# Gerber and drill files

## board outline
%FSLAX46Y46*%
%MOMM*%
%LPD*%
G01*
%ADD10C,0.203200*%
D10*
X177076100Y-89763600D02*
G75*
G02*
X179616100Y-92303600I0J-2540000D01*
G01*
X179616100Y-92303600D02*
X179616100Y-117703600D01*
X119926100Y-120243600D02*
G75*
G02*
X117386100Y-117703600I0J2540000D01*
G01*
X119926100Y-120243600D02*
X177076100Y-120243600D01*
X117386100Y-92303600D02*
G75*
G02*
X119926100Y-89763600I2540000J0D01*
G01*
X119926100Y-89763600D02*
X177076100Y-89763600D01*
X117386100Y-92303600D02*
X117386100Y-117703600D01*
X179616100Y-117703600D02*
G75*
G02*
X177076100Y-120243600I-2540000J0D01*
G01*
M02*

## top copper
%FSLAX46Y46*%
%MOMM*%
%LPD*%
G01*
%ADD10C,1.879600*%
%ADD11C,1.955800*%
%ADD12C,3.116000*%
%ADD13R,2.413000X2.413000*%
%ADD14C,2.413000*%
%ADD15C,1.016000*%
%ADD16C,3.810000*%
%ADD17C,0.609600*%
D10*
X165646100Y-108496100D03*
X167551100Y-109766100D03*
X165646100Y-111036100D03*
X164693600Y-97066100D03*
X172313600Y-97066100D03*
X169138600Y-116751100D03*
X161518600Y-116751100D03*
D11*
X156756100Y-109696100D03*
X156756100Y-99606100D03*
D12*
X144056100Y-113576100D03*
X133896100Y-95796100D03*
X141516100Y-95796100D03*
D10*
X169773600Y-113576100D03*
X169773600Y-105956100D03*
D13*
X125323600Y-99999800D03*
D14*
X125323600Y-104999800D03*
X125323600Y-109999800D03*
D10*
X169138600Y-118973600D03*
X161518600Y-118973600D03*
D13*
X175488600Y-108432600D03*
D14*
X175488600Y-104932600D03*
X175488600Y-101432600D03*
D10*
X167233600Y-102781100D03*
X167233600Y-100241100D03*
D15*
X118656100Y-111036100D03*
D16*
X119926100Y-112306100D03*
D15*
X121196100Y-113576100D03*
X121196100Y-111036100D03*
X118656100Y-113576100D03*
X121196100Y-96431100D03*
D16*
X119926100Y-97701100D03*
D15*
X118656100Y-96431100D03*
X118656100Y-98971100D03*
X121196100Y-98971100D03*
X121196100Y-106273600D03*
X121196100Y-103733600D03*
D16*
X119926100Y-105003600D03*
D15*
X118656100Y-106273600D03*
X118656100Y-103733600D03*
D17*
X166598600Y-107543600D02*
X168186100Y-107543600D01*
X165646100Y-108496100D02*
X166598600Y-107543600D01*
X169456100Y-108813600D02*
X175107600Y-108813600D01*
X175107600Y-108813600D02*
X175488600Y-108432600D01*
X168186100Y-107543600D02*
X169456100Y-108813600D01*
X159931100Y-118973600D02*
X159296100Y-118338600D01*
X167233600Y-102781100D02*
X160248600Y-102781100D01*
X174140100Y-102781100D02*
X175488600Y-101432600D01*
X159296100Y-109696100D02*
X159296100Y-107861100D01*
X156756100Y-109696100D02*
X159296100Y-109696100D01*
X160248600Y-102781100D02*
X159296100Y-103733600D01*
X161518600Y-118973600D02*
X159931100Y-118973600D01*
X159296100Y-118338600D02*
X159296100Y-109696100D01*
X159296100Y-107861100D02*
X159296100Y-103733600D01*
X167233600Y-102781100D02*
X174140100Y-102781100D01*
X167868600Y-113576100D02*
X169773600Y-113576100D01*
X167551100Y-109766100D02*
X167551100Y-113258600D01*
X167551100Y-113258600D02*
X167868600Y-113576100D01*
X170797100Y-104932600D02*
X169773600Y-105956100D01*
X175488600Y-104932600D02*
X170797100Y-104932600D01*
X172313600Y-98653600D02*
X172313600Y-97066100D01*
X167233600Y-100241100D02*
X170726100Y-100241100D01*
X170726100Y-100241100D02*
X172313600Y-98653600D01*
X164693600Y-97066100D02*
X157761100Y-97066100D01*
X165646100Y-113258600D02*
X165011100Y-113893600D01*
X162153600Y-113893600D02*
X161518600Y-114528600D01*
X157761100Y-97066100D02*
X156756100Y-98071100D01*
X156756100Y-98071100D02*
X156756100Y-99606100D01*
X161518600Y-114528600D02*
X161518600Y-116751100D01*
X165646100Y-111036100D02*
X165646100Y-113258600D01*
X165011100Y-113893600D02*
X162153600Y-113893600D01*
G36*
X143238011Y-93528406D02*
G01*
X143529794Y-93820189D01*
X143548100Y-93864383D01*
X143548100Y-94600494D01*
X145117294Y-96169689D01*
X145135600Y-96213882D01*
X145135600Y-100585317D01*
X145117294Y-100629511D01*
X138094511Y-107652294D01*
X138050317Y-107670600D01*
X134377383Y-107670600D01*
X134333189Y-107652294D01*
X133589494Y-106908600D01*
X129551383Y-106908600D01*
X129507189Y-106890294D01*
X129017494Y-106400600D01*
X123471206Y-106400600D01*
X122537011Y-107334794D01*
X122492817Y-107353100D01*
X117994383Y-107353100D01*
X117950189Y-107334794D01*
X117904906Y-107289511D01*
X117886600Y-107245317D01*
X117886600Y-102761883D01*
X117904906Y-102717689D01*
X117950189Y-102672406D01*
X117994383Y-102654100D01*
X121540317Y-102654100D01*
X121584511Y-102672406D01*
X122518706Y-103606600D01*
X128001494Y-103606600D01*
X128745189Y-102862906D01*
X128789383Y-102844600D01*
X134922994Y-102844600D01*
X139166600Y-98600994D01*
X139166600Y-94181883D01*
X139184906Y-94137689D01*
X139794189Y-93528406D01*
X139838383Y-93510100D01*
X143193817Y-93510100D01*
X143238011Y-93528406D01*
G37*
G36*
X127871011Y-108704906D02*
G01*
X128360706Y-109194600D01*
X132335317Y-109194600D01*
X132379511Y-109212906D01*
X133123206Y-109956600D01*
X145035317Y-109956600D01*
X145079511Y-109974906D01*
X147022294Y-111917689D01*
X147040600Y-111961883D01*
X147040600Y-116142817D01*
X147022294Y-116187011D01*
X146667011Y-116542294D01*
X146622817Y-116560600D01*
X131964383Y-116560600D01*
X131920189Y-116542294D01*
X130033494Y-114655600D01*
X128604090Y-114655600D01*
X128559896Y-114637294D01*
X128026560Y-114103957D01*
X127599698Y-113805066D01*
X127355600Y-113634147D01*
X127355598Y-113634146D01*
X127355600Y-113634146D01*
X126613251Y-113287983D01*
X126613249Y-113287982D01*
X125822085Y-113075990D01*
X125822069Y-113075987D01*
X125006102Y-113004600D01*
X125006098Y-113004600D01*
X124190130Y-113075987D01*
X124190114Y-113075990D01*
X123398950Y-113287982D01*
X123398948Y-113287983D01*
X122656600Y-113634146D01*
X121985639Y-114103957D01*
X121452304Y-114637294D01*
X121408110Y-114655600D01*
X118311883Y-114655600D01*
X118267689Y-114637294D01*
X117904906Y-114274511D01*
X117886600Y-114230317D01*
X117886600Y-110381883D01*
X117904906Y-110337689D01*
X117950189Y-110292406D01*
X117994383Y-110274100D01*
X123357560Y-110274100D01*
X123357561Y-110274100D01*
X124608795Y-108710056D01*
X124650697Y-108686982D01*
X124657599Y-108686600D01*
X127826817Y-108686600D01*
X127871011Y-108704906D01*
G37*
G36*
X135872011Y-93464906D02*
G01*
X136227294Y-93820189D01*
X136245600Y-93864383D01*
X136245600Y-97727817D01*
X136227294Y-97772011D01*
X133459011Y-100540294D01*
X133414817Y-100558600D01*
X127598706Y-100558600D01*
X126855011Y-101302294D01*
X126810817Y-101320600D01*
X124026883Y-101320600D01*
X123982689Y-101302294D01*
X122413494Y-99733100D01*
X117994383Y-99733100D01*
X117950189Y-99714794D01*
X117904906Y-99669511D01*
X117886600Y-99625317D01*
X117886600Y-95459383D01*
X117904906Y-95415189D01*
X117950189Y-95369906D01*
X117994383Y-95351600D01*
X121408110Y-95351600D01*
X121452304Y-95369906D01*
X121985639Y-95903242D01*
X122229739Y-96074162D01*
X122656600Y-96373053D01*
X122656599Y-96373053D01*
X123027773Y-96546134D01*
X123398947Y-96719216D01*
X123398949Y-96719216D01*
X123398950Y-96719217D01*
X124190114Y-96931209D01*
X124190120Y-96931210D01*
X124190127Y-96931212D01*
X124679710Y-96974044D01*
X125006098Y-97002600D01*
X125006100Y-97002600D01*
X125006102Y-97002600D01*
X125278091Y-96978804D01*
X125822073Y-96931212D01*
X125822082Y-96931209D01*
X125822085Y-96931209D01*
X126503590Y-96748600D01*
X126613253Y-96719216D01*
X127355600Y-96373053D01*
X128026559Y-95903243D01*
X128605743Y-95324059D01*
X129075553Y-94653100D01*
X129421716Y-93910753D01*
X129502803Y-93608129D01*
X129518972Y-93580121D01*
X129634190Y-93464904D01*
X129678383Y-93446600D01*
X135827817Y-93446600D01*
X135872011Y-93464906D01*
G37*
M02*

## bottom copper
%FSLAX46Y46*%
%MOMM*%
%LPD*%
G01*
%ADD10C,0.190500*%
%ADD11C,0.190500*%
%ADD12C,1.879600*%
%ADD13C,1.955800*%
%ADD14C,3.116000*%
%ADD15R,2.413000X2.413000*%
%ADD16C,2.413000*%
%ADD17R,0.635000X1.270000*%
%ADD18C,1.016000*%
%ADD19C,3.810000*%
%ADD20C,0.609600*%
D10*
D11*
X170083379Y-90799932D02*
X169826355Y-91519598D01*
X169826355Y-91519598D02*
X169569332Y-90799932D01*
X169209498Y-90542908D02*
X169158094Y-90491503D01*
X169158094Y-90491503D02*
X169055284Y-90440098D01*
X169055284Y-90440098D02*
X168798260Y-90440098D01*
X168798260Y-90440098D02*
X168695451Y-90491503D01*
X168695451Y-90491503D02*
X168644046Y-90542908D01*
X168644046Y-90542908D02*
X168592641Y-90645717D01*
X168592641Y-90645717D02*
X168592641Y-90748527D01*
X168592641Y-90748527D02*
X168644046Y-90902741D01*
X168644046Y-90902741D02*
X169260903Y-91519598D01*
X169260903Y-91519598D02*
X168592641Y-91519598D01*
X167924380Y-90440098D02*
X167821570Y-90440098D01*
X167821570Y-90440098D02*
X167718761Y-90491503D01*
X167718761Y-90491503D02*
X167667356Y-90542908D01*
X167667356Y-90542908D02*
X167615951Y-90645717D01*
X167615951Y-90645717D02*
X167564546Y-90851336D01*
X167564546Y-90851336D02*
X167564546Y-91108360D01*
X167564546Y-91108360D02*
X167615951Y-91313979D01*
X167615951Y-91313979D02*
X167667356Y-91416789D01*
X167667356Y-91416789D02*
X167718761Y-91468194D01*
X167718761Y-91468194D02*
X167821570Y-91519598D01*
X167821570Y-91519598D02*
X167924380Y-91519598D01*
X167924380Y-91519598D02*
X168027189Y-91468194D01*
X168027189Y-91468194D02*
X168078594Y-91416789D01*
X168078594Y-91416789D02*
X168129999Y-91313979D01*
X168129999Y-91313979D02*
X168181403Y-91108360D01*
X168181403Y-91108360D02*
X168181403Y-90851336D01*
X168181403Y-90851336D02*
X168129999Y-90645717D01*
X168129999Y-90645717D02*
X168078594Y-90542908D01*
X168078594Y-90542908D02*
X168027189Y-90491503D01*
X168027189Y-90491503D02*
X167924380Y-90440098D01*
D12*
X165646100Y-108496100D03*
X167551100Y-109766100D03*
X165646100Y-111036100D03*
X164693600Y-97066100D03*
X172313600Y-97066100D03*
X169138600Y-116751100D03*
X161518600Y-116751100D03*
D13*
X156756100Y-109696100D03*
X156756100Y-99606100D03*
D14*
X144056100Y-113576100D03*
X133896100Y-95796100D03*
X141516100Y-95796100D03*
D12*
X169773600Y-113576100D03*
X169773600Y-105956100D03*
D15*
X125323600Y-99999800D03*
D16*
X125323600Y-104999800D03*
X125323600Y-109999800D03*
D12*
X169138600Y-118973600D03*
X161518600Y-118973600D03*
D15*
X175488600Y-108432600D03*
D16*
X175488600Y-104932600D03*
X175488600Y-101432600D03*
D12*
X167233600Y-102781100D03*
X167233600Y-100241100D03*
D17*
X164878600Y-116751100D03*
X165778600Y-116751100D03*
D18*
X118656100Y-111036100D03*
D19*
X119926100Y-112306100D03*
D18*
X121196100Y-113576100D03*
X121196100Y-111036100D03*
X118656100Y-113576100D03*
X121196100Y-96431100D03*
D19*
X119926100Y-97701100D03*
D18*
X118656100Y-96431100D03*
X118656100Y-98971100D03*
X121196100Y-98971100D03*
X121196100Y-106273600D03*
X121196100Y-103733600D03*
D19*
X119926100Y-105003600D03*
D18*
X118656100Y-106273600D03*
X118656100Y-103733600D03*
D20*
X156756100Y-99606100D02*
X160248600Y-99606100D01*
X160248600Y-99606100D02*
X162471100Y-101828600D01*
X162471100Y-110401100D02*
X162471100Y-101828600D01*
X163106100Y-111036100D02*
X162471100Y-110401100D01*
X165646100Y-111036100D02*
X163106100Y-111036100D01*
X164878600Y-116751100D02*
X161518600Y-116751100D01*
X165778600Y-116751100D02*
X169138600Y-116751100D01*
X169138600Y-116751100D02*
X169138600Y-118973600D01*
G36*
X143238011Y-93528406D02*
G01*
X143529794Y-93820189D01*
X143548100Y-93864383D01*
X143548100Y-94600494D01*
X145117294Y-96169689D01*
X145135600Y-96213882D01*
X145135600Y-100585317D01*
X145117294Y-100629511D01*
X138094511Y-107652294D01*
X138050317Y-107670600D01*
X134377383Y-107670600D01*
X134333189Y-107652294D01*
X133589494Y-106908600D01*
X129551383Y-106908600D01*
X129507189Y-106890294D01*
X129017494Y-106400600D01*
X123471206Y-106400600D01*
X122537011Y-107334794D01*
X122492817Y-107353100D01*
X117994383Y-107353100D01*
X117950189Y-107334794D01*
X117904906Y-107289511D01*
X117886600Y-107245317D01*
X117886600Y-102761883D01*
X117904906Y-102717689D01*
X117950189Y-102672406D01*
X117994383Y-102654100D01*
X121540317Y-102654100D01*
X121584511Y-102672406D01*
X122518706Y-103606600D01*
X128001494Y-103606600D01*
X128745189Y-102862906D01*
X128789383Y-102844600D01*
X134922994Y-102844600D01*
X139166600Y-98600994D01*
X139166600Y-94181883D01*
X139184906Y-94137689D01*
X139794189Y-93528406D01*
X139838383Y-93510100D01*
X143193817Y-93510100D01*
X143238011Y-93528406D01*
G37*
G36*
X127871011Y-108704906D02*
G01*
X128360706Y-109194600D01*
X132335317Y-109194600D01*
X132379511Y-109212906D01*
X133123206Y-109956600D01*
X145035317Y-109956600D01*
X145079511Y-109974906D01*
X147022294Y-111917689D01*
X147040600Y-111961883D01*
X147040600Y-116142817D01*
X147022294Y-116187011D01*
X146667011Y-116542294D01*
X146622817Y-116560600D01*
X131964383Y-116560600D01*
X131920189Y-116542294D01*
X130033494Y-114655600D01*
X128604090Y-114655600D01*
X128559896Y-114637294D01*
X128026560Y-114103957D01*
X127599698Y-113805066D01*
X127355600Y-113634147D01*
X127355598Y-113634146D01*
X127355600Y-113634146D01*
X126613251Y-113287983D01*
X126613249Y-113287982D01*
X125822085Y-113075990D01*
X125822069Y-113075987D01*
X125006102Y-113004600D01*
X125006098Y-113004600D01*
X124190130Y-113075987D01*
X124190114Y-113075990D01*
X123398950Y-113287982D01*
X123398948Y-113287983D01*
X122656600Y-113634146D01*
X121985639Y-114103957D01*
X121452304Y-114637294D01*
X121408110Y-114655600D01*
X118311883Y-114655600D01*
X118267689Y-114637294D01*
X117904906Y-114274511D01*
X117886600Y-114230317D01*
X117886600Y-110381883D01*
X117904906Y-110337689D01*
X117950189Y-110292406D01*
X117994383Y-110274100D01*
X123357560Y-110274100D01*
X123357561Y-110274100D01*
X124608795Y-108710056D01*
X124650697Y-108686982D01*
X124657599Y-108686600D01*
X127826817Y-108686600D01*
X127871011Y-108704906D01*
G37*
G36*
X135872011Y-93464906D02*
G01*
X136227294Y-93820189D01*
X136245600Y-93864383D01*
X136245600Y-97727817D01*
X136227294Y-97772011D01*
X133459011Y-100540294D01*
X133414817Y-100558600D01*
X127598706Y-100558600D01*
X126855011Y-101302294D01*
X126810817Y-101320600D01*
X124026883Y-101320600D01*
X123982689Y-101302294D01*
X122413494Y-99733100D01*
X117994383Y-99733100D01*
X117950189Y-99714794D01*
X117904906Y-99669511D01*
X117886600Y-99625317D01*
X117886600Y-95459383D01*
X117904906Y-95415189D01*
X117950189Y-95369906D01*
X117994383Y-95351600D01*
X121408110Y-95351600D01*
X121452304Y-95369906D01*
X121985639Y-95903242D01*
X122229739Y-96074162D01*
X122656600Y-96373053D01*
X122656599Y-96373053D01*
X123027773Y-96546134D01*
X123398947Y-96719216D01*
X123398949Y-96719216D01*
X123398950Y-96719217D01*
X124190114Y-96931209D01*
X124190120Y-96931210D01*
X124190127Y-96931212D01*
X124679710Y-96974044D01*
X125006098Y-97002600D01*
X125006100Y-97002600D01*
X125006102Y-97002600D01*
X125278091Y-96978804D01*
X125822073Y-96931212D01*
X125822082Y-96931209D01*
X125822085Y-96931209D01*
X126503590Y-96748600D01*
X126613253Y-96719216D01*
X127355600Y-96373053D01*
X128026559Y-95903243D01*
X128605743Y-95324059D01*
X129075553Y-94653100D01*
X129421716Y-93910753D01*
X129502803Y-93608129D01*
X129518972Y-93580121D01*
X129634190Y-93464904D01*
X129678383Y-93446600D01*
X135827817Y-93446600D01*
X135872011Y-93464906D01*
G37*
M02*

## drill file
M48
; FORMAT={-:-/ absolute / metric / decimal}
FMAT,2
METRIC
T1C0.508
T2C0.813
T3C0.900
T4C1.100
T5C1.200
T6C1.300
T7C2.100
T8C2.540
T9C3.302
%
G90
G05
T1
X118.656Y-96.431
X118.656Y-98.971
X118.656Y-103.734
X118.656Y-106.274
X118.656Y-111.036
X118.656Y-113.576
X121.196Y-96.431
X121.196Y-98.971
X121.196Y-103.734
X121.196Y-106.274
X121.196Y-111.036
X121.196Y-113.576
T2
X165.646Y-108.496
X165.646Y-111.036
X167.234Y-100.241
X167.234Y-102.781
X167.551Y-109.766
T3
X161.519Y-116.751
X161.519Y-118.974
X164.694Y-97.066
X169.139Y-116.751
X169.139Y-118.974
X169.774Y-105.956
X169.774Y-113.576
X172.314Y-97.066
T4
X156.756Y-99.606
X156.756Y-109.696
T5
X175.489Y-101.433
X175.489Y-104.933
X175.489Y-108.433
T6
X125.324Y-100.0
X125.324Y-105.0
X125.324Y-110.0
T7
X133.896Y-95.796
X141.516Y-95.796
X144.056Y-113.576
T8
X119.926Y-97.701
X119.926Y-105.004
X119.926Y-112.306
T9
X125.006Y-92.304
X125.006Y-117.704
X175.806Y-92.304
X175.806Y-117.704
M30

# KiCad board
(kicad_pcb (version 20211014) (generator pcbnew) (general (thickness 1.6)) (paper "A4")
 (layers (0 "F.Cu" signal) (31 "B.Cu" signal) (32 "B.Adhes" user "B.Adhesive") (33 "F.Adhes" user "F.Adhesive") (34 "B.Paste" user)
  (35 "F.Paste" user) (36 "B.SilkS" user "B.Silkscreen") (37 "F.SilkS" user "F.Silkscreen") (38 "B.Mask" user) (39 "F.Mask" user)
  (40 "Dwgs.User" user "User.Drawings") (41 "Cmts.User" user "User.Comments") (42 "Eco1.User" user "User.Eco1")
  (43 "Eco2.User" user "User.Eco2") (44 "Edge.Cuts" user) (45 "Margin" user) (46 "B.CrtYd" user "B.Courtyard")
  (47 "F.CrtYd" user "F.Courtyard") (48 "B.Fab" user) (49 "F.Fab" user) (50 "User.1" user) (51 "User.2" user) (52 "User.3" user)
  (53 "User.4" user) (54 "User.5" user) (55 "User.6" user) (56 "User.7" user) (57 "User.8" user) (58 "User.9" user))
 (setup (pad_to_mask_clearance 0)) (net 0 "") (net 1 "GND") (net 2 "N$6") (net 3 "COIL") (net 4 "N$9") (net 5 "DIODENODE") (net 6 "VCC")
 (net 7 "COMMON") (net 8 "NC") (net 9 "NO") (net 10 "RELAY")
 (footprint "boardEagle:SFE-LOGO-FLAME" (layer "F.Cu") (at 167.8686 94.2086)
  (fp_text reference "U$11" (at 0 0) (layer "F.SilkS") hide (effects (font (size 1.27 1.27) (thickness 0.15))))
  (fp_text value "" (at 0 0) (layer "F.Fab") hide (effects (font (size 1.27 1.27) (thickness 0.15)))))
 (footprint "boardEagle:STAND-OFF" (layer "F.Cu") (at 125.0061 117.7036)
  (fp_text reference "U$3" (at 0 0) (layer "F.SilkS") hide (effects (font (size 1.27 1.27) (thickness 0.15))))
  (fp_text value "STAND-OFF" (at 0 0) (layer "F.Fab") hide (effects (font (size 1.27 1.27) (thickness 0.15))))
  (pad "" np_thru_hole circle (at 0 0) (size 3.302 3.302) (drill 3.302) (layers *.Cu *.Mask)))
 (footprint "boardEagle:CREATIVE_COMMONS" (layer "F.Cu") (at 116.2431 133.3246)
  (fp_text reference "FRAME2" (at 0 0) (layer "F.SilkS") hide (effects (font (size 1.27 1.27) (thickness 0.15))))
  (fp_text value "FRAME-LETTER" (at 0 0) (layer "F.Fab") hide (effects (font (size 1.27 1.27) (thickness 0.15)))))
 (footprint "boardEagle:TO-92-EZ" (layer "F.Cu") (at 165.6461 109.7661 -90)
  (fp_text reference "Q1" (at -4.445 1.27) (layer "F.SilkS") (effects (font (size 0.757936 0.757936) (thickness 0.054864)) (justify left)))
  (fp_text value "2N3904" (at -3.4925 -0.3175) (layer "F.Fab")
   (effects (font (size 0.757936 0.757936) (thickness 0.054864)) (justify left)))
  (pad "1" thru_hole circle (at -1.27 0 270) (size 1.8796 1.8796) (drill 0.8128) (layers *.Cu) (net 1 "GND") (solder_mask_margin 0.1016))
  (pad "2" thru_hole circle (at 0 -1.905 270) (size 1.8796 1.8796) (drill 0.8128) (layers *.Cu) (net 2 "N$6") (solder_mask_margin 0.1016))
  (pad "3" thru_hole circle (at 1.27 0 270) (size 1.8796 1.8796) (drill 0.8128) (layers *.Cu) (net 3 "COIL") (solder_mask_margin 0.1016)))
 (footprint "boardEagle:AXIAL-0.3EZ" (layer "F.Cu") (at 168.5036 97.0661)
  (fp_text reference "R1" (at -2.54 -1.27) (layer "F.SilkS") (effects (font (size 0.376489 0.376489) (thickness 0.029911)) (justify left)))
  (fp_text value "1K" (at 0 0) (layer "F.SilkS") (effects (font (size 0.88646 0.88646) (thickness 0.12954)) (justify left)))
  (pad "P$1" thru_hole circle (at -3.81 0) (size 1.8796 1.8796) (drill 0.9) (layers *.Cu) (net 3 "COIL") (solder_mask_margin 0.1016))
  (pad "P$2" thru_hole circle (at 3.81 0) (size 1.8796 1.8796) (drill 0.9) (layers *.Cu) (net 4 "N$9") (solder_mask_margin 0.1016)))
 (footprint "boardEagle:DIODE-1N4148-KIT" (layer "F.Cu") (at 165.3286 116.7511 180)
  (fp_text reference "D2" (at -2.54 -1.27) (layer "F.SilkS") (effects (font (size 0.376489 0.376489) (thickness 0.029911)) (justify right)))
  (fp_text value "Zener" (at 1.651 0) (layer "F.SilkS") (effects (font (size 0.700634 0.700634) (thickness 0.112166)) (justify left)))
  (pad "A" thru_hole circle (at -3.81 0 180) (size 1.8796 1.8796) (drill 0.9) (layers *.Cu) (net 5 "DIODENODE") (solder_mask_margin 0.1016))
  (pad "C" thru_hole circle (at 3.81 0 180) (size 1.8796 1.8796) (drill 0.9) (layers *.Cu) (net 3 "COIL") (solder_mask_margin 0.1016)))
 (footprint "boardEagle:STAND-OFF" (layer "F.Cu") (at 175.8061 117.7036)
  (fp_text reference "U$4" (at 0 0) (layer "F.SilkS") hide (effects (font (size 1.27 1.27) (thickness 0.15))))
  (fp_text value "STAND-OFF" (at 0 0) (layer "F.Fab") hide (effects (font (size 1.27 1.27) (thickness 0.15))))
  (pad "" np_thru_hole circle (at 0 0) (size 3.302 3.302) (drill 3.302) (layers *.Cu *.Mask)))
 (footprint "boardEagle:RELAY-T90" (layer "F.Cu") (at 156.7561 95.7961)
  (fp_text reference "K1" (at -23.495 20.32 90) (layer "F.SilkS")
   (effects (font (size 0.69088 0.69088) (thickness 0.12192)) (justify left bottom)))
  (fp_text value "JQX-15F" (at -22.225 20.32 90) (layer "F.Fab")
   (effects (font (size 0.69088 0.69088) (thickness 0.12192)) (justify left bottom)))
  (pad "COIL1" thru_hole circle (at 0 13.9 90) (size 1.9558 1.9558) (drill 1.1) (layers *.Cu *.Mask) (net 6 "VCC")
   (solder_mask_margin 0.1016))
  (pad "COIL2" thru_hole circle (at 0 3.81 90) (size 1.9558 1.9558) (drill 1.1) (layers *.Cu *.Mask) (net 3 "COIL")
   (solder_mask_margin 0.1016))
  (pad "MAIN" thru_hole circle (at -12.7 17.78 90) (size 3.116 3.116) (drill 2.1) (layers *.Cu *.Mask) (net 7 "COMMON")
   (solder_mask_margin 0.1016))
  (pad "NC" thru_hole circle (at -22.86 0 90) (size 3.116 3.116) (drill 2.1) (layers *.Cu *.Mask) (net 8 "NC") (solder_mask_margin 0.1016))
  (pad "NO" thru_hole circle (at -15.24 0 90) (size 3.116 3.116) (drill 2.1) (layers *.Cu *.Mask) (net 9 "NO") (solder_mask_margin 0.1016)))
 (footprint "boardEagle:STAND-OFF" (layer "F.Cu") (at 175.8061 92.3036)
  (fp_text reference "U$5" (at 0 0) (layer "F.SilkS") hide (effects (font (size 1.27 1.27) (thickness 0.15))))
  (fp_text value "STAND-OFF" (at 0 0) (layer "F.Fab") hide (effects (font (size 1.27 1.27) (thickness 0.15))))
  (pad "" np_thru_hole circle (at 0 0) (size 3.302 3.302) (drill 3.302) (layers *.Cu *.Mask)))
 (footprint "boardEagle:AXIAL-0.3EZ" (layer "F.Cu") (at 169.7736 109.7661 90)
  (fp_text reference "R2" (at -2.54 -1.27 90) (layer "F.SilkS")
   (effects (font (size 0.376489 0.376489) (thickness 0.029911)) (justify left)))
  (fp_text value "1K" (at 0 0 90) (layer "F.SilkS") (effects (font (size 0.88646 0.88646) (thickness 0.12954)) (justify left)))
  (pad "P$1" thru_hole circle (at -3.81 0 90) (size 1.8796 1.8796) (drill 0.9) (layers *.Cu) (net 2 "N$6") (solder_mask_margin 0.1016))
  (pad "P$2" thru_hole circle (at 3.81 0 90) (size 1.8796 1.8796) (drill 0.9) (layers *.Cu) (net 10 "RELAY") (solder_mask_margin 0.1016)))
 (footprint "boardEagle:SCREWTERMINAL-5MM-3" (layer "F.Cu") (at 125.3236 99.9998 -90)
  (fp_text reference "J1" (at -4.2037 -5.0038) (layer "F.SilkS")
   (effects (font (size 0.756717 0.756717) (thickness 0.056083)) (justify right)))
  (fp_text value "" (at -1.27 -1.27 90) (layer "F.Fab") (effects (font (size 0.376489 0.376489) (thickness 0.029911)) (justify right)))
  (pad "1" thru_hole rect (at 0 0 270) (size 2.413 2.413) (drill 1.3) (layers *.Cu *.Mask) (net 8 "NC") (solder_mask_margin 0.1016))
  (pad "2" thru_hole circle (at 5 0 270) (size 2.413 2.413) (drill 1.3) (layers *.Cu *.Mask) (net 9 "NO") (solder_mask_margin 0.1016))
  (pad "3" thru_hole circle (at 10 0 270) (size 2.413 2.413) (drill 1.3) (layers *.Cu *.Mask) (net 7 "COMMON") (solder_mask_margin 0.1016)))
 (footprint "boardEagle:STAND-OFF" (layer "F.Cu") (at 125.0061 92.3036)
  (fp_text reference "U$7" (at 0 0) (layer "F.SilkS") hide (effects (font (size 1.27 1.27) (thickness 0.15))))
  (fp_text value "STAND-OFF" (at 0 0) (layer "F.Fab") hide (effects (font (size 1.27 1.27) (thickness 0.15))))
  (pad "" np_thru_hole circle (at 0 0) (size 3.302 3.302) (drill 3.302) (layers *.Cu *.Mask)))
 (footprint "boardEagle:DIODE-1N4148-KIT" (layer "F.Cu") (at 165.3286 118.9736 180)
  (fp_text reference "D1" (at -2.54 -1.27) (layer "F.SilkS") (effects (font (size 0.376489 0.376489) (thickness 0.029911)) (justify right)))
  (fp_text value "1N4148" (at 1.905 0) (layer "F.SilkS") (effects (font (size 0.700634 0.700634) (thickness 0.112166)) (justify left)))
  (pad "A" thru_hole circle (at -3.81 0 180) (size 1.8796 1.8796) (drill 0.9) (layers *.Cu) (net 5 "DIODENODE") (solder_mask_margin 0.1016))
  (pad "C" thru_hole circle (at 3.81 0 180) (size 1.8796 1.8796) (drill 0.9) (layers *.Cu) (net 6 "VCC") (solder_mask_margin 0.1016)))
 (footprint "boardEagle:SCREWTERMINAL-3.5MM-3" (layer "F.Cu") (at 175.4886 108.4326 90)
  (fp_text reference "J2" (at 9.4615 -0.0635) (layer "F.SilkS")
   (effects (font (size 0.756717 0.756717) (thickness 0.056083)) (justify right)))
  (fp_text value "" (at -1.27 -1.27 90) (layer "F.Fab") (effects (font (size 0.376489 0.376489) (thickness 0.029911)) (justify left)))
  (pad "1" thru_hole rect (at 0 0 90) (size 2.413 2.413) (drill 1.2) (layers *.Cu *.Mask) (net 1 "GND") (solder_mask_margin 0.1016))
  (pad "2" thru_hole circle (at 3.5 0 90) (size 2.413 2.413) (drill 1.2) (layers *.Cu *.Mask) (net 10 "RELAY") (solder_mask_margin 0.1016))
  (pad "3" thru_hole circle (at 7 0 90) (size 2.413 2.413) (drill 1.2) (layers *.Cu *.Mask) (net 6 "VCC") (solder_mask_margin 0.1016)))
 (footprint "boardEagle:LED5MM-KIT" (layer "F.Cu") (at 167.2336 101.5111 90)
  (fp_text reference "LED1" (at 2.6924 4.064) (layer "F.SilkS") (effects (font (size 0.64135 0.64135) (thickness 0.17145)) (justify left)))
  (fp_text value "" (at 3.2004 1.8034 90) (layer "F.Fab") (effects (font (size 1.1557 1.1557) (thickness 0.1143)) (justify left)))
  (pad "A" thru_hole circle (at -1.27 0 90) (size 1.8796 1.8796) (drill 0.8128) (layers *.Cu) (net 6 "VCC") (solder_mask_margin 0.1016))
  (pad "K" thru_hole circle (at 1.27 0 90) (size 1.8796 1.8796) (drill 0.8128) (layers *.Cu) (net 4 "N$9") (solder_mask_margin 0.1016)))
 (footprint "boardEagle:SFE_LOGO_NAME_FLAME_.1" (layer "B.Cu") (at 142.3416 117.3861 180)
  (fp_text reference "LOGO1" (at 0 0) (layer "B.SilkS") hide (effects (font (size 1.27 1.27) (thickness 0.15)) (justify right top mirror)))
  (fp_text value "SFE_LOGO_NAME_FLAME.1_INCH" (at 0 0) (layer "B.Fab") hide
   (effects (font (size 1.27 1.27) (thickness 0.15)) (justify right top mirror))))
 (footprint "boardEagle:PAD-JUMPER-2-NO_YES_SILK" (layer "B.Cu") (at 165.3286 116.7511)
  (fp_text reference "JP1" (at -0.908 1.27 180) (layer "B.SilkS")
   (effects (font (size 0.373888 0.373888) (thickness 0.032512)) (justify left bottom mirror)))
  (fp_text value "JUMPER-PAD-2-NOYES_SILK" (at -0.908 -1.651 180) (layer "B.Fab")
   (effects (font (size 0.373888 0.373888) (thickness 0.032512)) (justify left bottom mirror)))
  (pad "1" smd rect (at -0.45 0) (size 0.635 1.27) (layers "B.Cu" "B.Mask") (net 3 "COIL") (solder_mask_margin 0.1016))
  (pad "2" smd rect (at 0.45 0) (size 0.635 1.27) (layers "B.Cu" "B.Mask") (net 5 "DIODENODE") (solder_mask_margin 0.1016)))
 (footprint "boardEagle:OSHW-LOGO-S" (layer "B.Cu") (at 169.1386 93.5736 180)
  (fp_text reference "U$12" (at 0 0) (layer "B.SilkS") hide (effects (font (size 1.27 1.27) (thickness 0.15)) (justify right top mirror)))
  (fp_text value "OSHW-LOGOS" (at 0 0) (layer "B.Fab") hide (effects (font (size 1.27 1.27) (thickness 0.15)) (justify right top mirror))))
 (gr_arc (start 177.0761 89.7636) (mid 178.872151 90.507549) (end 179.6161 92.3036) (layer "Edge.Cuts") (width 0.2032))
 (gr_line (start 179.6161 92.3036) (end 179.6161 117.7036) (layer "Edge.Cuts") (width 0.2032))
 (gr_arc (start 119.9261 120.2436) (mid 118.130049 119.499651) (end 117.3861 117.7036) (layer "Edge.Cuts") (width 0.2032))
 (gr_line (start 119.9261 120.2436) (end 177.0761 120.2436) (layer "Edge.Cuts") (width 0.2032))
 (gr_arc (start 117.3861 92.3036) (mid 118.130049 90.507549) (end 119.9261 89.7636) (layer "Edge.Cuts") (width 0.2032))
 (gr_line (start 119.9261 89.7636) (end 177.0761 89.7636) (layer "Edge.Cuts") (width 0.2032))
 (gr_line (start 117.3861 92.3036) (end 117.3861 117.7036) (layer "Edge.Cuts") (width 0.2032))
 (gr_arc (start 179.6161 117.7036) (mid 178.872151 119.499651) (end 177.0761 120.2436) (layer "Edge.Cuts") (width 0.2032))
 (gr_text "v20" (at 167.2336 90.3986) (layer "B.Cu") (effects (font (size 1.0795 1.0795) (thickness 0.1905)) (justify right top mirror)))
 (segment (start 166.5986 107.5436) (end 168.1861 107.5436) (width 0.6096) (layer "F.Cu") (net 1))
 (segment (start 165.6461 108.4961) (end 166.5986 107.5436) (width 0.6096) (layer "F.Cu") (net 1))
 (segment (start 169.4561 108.8136) (end 175.1076 108.8136) (width 0.6096) (layer "F.Cu") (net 1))
 (segment (start 175.1076 108.8136) (end 175.4886 108.4326) (width 0.6096) (layer "F.Cu") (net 1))
 (segment (start 168.1861 107.5436) (end 169.4561 108.8136) (width 0.6096) (layer "F.Cu") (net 1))
 (segment (start 159.9311 118.9736) (end 159.2961 118.3386) (width 0.6096) (layer "F.Cu") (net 6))
 (segment (start 167.2336 102.7811) (end 160.2486 102.7811) (width 0.6096) (layer "F.Cu") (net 6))
 (segment (start 174.1401 102.7811) (end 175.4886 101.4326) (width 0.6096) (layer "F.Cu") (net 6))
 (segment (start 159.2961 109.6961) (end 159.2961 107.8611) (width 0.6096) (layer "F.Cu") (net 6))
 (segment (start 156.7561 109.6961) (end 159.2961 109.6961) (width 0.6096) (layer "F.Cu") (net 6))
 (segment (start 160.2486 102.7811) (end 159.2961 103.7336) (width 0.6096) (layer "F.Cu") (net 6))
 (segment (start 161.5186 118.9736) (end 159.9311 118.9736) (width 0.6096) (layer "F.Cu") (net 6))
 (segment (start 159.2961 118.3386) (end 159.2961 109.6961) (width 0.6096) (layer "F.Cu") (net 6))
 (segment (start 159.2961 107.8611) (end 159.2961 103.7336) (width 0.6096) (layer "F.Cu") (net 6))
 (segment (start 167.2336 102.7811) (end 174.1401 102.7811) (width 0.6096) (layer "F.Cu") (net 6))
 (segment (start 167.8686 113.5761) (end 169.7736 113.5761) (width 0.6096) (layer "F.Cu") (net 2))
 (segment (start 167.5511 109.7661) (end 167.5511 113.2586) (width 0.6096) (layer "F.Cu") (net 2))
 (segment (start 167.5511 113.2586) (end 167.8686 113.5761) (width 0.6096) (layer "F.Cu") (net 2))
 (segment (start 170.7971 104.9326) (end 169.7736 105.9561) (width 0.6096) (layer "F.Cu") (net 10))
 (segment (start 175.4886 104.9326) (end 170.7971 104.9326) (width 0.6096) (layer "F.Cu") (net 10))
 (segment (start 172.3136 98.6536) (end 172.3136 97.0661) (width 0.6096) (layer "F.Cu") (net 4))
 (segment (start 167.2336 100.2411) (end 170.7261 100.2411) (width 0.6096) (layer "F.Cu") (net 4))
 (segment (start 170.7261 100.2411) (end 172.3136 98.6536) (width 0.6096) (layer "F.Cu") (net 4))
 (segment (start 164.6936 97.0661) (end 157.7611 97.0661) (width 0.6096) (layer "F.Cu") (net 3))
 (segment (start 165.6461 113.2586) (end 165.0111 113.8936) (width 0.6096) (layer "F.Cu") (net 3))
 (segment (start 162.1536 113.8936) (end 161.5186 114.5286) (width 0.6096) (layer "F.Cu") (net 3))
 (segment (start 157.7611 97.0661) (end 156.7561 98.0711) (width 0.6096) (layer "F.Cu") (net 3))
 (segment (start 156.7561 98.0711) (end 156.7561 99.6061) (width 0.6096) (layer "F.Cu") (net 3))
 (segment (start 161.5186 114.5286) (end 161.5186 116.7511) (width 0.6096) (layer "F.Cu") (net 3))
 (segment (start 165.6461 111.0361) (end 165.6461 113.2586) (width 0.6096) (layer "F.Cu") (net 3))
 (segment (start 165.0111 113.8936) (end 162.1536 113.8936) (width 0.6096) (layer "F.Cu") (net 3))
 (segment (start 156.7561 99.6061) (end 160.2486 99.6061) (width 0.6096) (layer "B.Cu") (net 3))
 (segment (start 160.2486 99.6061) (end 162.4711 101.8286) (width 0.6096) (layer "B.Cu") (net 3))
 (segment (start 162.4711 110.4011) (end 162.4711 101.8286) (width 0.6096) (layer "B.Cu") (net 3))
 (segment (start 163.1061 111.0361) (end 162.4711 110.4011) (width 0.6096) (layer "B.Cu") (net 3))
 (segment (start 165.6461 111.0361) (end 163.1061 111.0361) (width 0.6096) (layer "B.Cu") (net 3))
 (segment (start 164.8786 116.7511) (end 161.5186 116.7511) (width 0.6096) (layer "B.Cu") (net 3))
 (via (at 118.6561 111.0361) (size 1.016) (drill 0.508) (layers "F.Cu" "B.Cu") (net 7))
 (via (at 119.9261 112.3061) (size 3.81) (drill 2.54) (layers "F.Cu" "B.Cu") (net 7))
 (via (at 121.1961 113.5761) (size 1.016) (drill 0.508) (layers "F.Cu" "B.Cu") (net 7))
 (via (at 121.1961 111.0361) (size 1.016) (drill 0.508) (layers "F.Cu" "B.Cu") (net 7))
 (via (at 118.6561 113.5761) (size 1.016) (drill 0.508) (layers "F.Cu" "B.Cu") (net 7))
 (via (at 121.1961 96.4311) (size 1.016) (drill 0.508) (layers "F.Cu" "B.Cu") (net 8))
 (via (at 119.9261 97.7011) (size 3.81) (drill 2.54) (layers "F.Cu" "B.Cu") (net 8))
 (via (at 118.6561 96.4311) (size 1.016) (drill 0.508) (layers "F.Cu" "B.Cu") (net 8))
 (via (at 118.6561 98.9711) (size 1.016) (drill 0.508) (layers "F.Cu" "B.Cu") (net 8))
 (via (at 121.1961 98.9711) (size 1.016) (drill 0.508) (layers "F.Cu" "B.Cu") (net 8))
 (via (at 121.1961 106.2736) (size 1.016) (drill 0.508) (layers "F.Cu" "B.Cu") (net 9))
 (via (at 121.1961 103.7336) (size 1.016) (drill 0.508) (layers "F.Cu" "B.Cu") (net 9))
 (via (at 119.9261 105.0036) (size 3.81) (drill 2.54) (layers "F.Cu" "B.Cu") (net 9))
 (via (at 118.6561 106.2736) (size 1.016) (drill 0.508) (layers "F.Cu" "B.Cu") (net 9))
 (via (at 118.6561 103.7336) (size 1.016) (drill 0.508) (layers "F.Cu" "B.Cu") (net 9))
 (segment (start 165.7786 116.7511) (end 169.1386 116.7511) (width 0.6096) (layer "B.Cu") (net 5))
 (segment (start 169.1386 116.7511) (end 169.1386 118.9736) (width 0.6096) (layer "B.Cu") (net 5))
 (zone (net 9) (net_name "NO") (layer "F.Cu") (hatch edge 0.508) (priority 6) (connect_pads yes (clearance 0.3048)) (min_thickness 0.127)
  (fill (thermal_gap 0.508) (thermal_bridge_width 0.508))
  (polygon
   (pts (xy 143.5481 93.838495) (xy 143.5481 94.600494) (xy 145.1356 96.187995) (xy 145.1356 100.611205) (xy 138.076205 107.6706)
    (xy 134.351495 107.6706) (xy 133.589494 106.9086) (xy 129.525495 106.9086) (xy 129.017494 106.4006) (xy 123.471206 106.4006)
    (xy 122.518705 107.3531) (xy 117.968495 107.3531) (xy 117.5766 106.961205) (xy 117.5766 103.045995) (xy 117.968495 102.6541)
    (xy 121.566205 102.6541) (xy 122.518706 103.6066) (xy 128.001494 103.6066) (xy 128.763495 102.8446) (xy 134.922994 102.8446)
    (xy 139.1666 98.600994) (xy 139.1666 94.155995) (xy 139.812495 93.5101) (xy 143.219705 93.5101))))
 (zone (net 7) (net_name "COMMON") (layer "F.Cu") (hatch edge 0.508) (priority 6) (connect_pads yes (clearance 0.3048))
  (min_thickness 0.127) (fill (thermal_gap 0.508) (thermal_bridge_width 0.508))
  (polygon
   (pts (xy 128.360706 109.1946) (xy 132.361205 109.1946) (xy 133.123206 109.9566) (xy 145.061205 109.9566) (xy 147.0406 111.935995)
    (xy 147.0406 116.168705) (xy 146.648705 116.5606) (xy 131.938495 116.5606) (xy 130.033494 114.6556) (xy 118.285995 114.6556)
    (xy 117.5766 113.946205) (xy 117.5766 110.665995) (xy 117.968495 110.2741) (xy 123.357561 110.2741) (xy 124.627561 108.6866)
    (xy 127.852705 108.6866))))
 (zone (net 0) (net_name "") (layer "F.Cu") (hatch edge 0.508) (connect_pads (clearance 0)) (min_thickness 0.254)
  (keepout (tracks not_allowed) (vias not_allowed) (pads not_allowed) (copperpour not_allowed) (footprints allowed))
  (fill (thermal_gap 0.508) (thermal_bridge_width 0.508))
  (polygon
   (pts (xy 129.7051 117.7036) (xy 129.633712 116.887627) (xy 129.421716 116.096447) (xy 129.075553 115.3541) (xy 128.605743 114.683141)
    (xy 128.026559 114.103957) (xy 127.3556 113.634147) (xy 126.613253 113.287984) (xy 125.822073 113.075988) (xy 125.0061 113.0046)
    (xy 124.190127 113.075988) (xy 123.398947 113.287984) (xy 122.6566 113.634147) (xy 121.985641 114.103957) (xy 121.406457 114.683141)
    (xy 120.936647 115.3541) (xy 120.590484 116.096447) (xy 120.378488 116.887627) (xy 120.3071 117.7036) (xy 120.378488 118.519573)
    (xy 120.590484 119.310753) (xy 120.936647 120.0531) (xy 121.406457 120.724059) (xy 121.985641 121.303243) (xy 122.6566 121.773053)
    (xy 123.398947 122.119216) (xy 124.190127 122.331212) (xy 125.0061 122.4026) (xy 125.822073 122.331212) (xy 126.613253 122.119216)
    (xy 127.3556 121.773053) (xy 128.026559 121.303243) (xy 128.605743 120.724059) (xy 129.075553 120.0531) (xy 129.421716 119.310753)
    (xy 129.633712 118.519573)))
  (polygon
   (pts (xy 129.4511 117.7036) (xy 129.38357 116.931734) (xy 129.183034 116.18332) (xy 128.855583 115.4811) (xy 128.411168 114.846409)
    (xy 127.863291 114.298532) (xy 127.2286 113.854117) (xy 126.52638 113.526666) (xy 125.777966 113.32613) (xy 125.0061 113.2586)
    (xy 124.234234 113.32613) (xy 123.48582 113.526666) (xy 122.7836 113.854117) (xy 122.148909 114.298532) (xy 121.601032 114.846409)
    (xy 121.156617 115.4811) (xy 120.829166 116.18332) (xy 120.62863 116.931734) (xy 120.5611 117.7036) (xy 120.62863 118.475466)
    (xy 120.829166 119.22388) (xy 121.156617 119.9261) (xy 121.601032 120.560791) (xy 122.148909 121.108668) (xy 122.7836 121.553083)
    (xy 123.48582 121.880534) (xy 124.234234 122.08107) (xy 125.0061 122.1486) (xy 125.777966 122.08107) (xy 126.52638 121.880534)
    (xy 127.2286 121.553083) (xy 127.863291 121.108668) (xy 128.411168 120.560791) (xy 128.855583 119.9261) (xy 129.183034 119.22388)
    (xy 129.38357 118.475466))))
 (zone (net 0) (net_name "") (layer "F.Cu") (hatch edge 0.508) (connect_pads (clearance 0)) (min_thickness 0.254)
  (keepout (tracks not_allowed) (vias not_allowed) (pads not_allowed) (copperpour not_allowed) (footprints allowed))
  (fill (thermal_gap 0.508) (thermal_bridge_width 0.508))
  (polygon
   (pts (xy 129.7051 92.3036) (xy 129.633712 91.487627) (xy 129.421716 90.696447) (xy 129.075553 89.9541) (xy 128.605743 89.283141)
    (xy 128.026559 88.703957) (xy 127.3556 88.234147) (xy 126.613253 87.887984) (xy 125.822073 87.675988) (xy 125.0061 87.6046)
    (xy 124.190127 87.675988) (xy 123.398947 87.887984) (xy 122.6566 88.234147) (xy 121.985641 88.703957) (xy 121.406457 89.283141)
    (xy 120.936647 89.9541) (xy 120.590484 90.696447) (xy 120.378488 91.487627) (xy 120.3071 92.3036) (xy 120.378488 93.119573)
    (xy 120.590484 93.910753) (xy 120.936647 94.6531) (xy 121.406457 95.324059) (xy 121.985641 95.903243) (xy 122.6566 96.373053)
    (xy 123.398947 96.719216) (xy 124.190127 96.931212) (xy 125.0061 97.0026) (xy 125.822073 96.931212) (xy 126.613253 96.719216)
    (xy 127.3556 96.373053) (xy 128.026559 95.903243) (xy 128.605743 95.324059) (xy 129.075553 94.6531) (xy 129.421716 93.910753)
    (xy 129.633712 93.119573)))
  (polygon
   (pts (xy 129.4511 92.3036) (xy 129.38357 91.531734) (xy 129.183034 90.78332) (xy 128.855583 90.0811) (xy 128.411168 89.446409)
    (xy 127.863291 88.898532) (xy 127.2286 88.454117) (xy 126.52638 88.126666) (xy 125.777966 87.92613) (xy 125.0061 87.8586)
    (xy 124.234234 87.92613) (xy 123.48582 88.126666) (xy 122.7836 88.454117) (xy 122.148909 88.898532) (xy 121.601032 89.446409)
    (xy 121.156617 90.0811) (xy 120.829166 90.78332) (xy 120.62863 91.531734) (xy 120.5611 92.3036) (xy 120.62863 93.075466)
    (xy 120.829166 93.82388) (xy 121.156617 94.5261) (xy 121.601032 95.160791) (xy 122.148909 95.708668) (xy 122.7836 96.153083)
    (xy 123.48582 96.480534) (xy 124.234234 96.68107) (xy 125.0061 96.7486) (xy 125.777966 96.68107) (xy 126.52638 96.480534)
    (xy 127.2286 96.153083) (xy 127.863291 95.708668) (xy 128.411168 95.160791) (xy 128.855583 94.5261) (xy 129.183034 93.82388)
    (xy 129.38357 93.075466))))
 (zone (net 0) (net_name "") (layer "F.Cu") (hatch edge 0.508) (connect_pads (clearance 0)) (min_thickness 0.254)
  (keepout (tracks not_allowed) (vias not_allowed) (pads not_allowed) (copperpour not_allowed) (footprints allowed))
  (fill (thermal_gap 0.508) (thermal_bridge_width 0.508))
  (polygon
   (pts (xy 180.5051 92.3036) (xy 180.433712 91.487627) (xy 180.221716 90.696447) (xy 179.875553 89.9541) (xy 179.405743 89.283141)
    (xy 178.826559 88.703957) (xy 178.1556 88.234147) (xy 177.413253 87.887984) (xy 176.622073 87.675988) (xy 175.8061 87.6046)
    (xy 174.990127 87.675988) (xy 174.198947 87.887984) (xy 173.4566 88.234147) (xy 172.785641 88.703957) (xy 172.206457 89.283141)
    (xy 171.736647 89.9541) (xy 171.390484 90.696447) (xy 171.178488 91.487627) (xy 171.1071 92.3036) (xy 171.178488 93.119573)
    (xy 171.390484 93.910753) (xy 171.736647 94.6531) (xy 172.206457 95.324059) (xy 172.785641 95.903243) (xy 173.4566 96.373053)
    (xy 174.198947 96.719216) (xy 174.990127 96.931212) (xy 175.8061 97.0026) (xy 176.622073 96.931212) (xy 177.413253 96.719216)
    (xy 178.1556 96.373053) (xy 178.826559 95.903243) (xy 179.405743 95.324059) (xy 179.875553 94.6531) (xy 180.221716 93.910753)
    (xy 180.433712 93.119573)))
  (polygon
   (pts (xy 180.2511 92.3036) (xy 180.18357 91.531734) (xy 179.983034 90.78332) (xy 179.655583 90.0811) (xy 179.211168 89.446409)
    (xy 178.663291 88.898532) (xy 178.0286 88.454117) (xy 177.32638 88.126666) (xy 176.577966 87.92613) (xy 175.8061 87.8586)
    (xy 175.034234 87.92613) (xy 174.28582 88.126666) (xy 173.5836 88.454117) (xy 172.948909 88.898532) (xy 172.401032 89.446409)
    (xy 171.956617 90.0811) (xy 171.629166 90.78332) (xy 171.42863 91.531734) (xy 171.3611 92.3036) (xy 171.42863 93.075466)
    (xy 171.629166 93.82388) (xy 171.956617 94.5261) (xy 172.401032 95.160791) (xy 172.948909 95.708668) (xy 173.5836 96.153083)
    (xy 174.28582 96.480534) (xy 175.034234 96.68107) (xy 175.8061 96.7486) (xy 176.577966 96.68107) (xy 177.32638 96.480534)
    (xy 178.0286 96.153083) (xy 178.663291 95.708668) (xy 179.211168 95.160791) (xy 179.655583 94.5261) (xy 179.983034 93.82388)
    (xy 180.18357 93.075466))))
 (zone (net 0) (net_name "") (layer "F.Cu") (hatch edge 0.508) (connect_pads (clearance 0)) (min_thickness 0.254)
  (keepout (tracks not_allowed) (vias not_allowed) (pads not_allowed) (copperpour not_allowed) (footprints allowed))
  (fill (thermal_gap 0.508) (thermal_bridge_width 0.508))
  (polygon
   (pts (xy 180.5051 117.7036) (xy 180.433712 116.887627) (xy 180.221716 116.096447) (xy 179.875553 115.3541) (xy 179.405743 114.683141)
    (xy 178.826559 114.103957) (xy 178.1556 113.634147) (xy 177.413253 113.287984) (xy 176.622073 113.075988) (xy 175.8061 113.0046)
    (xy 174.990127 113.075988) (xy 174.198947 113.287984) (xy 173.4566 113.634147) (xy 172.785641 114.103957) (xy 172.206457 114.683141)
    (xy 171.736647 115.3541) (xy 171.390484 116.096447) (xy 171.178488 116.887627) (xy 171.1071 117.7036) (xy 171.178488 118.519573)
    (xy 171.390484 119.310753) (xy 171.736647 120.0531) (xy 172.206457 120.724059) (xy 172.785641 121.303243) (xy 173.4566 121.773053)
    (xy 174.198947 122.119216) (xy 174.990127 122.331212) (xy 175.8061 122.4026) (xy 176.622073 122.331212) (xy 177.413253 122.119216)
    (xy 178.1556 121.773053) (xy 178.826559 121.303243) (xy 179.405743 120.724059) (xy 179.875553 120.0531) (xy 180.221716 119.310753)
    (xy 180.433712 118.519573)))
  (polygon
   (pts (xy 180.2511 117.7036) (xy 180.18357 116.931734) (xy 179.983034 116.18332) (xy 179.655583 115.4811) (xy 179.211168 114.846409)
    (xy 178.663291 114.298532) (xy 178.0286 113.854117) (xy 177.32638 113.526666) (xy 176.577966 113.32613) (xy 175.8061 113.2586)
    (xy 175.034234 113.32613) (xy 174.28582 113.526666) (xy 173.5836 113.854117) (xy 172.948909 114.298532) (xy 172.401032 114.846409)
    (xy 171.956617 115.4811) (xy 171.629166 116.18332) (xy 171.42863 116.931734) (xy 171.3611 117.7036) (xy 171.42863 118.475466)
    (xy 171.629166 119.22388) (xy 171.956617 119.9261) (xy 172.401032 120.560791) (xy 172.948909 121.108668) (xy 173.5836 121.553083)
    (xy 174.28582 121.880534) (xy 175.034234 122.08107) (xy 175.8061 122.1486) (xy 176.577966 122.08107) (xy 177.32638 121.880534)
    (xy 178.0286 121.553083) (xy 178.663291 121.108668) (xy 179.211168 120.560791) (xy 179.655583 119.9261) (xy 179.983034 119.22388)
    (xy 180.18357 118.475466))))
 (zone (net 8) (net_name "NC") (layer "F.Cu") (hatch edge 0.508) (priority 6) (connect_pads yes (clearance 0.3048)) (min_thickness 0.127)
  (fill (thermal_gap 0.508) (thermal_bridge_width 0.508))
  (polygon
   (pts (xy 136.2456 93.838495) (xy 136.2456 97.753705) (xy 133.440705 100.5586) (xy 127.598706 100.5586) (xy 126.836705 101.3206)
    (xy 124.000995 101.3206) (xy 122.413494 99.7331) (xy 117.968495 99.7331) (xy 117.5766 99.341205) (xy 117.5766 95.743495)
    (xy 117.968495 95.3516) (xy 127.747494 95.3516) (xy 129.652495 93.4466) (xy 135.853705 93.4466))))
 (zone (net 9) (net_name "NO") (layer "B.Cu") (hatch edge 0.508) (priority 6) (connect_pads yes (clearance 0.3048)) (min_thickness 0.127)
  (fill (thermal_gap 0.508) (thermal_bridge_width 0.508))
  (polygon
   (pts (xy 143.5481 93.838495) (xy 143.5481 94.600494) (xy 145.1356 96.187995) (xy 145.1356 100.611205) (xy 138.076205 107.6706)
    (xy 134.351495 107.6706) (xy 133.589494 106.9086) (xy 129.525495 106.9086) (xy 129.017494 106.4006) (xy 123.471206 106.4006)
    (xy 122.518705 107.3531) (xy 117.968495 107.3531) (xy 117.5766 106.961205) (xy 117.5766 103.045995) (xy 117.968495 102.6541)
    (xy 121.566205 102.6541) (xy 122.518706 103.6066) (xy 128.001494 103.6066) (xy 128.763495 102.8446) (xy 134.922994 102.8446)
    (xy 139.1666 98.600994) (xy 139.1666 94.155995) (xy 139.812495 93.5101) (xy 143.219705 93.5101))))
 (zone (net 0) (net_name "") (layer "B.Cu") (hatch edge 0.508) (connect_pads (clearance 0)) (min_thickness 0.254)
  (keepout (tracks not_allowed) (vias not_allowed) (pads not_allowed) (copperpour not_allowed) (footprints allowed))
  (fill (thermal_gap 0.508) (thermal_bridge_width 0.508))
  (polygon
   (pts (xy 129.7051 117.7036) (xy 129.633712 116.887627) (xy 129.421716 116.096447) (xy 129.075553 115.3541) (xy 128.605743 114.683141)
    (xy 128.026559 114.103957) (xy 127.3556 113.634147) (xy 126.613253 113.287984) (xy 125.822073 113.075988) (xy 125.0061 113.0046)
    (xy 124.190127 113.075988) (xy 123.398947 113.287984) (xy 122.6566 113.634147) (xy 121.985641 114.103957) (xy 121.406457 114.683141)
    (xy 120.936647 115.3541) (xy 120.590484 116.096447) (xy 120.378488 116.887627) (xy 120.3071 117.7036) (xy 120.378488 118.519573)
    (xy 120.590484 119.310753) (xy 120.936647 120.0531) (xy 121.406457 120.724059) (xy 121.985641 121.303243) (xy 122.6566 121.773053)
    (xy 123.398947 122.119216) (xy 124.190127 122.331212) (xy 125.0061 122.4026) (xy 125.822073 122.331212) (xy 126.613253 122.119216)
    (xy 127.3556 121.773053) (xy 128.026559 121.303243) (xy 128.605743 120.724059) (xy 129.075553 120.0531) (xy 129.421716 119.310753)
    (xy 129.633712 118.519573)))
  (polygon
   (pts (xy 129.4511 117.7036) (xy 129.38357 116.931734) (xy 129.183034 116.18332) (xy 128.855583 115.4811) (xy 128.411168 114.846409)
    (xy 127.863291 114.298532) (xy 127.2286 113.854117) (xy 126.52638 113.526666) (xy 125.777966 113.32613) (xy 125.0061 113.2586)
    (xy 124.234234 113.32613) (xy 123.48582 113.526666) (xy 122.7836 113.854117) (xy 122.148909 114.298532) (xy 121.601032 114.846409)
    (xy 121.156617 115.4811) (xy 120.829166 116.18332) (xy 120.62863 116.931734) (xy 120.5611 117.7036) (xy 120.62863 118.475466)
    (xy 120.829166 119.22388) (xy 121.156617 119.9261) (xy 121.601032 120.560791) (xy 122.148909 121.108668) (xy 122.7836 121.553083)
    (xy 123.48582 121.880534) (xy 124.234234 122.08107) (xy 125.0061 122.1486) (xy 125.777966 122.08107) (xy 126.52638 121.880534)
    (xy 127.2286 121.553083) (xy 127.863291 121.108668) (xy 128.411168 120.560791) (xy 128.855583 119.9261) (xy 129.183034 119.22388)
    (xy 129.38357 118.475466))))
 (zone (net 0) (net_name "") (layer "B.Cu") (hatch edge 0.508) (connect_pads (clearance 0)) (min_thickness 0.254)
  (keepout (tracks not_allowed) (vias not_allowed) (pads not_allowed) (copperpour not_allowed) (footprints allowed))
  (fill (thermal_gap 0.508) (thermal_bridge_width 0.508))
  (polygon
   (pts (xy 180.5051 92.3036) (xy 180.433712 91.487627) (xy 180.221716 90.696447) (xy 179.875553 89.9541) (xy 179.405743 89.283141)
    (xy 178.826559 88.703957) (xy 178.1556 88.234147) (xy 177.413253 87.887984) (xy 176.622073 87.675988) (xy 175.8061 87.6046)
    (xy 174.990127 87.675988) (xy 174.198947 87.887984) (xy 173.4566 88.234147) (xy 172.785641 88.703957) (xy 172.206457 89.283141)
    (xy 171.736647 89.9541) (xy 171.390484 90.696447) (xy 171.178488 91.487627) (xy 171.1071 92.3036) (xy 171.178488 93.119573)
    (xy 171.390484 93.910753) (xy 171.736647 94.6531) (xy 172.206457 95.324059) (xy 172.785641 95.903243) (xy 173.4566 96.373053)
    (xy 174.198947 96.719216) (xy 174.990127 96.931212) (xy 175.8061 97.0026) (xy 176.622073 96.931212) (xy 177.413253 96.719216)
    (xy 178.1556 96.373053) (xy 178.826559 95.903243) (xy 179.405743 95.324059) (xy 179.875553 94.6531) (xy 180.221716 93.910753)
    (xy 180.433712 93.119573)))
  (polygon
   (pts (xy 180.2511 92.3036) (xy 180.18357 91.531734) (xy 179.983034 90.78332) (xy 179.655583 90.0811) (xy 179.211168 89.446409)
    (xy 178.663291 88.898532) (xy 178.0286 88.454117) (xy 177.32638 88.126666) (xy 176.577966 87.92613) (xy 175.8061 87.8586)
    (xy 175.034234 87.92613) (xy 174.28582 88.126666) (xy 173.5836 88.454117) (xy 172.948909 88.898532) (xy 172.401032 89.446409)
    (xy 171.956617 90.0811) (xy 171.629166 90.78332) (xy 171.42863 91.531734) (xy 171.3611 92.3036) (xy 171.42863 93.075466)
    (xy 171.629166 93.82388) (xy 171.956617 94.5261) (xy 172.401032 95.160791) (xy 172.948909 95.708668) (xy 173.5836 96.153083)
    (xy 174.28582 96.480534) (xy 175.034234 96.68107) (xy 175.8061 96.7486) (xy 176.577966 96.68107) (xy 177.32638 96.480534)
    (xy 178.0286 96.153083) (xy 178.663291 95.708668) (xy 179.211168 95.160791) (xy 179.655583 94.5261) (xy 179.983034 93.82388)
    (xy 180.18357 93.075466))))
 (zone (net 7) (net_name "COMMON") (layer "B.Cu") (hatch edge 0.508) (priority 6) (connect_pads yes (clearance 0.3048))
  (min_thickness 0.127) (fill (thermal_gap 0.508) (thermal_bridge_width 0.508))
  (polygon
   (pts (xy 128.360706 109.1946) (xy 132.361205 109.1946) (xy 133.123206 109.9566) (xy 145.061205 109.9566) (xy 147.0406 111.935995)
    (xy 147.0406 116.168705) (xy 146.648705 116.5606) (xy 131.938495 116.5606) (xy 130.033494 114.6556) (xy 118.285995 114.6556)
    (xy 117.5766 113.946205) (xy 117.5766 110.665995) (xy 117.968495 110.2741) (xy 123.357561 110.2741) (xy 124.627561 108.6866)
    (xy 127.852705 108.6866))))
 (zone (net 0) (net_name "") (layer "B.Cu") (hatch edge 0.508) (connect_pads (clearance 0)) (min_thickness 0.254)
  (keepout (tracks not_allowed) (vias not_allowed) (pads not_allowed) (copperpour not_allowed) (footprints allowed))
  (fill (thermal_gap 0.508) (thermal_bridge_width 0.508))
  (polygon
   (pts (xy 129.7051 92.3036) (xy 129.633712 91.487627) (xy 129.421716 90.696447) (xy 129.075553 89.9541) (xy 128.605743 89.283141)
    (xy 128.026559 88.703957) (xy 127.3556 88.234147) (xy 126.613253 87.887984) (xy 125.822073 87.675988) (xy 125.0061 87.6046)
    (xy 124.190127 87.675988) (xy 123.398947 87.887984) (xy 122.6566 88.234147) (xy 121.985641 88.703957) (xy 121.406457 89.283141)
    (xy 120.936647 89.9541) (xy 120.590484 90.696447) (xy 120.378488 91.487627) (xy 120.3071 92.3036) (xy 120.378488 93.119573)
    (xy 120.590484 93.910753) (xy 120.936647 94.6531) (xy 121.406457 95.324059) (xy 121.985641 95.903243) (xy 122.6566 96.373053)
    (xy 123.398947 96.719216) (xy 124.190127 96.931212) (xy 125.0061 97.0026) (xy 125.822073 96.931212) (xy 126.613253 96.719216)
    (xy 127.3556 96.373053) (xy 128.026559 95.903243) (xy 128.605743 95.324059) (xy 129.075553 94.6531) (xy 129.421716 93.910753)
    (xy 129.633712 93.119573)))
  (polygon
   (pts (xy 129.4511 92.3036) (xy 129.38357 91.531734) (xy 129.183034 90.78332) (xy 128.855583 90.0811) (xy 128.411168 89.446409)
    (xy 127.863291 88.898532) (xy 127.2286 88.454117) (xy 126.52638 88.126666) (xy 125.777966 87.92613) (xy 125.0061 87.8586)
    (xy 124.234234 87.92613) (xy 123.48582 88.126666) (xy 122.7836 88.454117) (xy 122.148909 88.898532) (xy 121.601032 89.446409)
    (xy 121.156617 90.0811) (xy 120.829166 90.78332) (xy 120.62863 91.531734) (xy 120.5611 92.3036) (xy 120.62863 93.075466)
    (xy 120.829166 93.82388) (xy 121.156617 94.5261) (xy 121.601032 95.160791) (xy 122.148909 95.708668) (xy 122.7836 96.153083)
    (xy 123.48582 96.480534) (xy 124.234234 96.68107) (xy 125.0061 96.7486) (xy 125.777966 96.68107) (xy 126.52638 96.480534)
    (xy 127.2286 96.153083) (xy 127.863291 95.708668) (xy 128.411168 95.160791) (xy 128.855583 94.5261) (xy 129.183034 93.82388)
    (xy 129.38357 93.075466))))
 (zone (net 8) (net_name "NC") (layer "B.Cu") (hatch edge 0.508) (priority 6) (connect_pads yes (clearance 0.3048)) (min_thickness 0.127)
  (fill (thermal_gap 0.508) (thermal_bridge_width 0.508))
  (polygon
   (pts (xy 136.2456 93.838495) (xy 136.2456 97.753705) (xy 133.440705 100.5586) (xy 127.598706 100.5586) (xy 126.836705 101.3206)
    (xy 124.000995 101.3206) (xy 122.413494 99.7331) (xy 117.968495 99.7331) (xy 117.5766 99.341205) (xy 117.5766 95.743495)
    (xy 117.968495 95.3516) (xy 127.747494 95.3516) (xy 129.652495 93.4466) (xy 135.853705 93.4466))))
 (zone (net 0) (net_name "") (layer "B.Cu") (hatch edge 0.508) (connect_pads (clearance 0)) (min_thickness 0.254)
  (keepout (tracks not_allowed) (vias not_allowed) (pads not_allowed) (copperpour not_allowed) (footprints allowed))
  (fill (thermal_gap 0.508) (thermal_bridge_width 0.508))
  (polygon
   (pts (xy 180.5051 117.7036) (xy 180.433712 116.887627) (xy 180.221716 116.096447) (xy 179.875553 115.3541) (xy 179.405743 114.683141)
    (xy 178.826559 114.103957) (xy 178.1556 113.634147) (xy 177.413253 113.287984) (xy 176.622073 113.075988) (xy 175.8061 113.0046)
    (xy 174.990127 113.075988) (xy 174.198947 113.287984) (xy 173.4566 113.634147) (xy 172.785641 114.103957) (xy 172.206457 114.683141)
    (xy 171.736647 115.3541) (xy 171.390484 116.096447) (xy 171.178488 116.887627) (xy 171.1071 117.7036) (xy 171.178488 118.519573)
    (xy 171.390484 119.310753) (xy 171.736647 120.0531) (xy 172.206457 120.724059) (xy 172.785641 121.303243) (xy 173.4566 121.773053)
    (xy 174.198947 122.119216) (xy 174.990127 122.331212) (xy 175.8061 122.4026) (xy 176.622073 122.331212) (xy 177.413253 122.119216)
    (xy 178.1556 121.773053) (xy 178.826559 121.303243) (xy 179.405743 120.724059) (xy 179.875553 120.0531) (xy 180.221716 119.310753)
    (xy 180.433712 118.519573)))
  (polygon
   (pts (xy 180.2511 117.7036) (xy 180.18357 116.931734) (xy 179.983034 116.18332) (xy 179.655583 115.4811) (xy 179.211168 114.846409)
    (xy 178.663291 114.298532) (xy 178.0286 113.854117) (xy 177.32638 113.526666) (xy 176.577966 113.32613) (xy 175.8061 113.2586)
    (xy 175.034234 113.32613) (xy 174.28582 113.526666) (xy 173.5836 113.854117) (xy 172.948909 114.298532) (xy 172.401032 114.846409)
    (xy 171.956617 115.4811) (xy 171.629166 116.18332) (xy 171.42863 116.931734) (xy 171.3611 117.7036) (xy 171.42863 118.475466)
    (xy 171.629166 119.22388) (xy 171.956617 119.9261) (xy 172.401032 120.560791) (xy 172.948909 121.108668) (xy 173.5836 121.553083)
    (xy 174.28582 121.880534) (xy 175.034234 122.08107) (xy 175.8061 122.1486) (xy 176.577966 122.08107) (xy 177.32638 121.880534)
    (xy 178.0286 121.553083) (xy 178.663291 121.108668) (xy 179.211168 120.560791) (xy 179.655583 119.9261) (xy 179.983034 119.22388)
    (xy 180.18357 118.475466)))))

